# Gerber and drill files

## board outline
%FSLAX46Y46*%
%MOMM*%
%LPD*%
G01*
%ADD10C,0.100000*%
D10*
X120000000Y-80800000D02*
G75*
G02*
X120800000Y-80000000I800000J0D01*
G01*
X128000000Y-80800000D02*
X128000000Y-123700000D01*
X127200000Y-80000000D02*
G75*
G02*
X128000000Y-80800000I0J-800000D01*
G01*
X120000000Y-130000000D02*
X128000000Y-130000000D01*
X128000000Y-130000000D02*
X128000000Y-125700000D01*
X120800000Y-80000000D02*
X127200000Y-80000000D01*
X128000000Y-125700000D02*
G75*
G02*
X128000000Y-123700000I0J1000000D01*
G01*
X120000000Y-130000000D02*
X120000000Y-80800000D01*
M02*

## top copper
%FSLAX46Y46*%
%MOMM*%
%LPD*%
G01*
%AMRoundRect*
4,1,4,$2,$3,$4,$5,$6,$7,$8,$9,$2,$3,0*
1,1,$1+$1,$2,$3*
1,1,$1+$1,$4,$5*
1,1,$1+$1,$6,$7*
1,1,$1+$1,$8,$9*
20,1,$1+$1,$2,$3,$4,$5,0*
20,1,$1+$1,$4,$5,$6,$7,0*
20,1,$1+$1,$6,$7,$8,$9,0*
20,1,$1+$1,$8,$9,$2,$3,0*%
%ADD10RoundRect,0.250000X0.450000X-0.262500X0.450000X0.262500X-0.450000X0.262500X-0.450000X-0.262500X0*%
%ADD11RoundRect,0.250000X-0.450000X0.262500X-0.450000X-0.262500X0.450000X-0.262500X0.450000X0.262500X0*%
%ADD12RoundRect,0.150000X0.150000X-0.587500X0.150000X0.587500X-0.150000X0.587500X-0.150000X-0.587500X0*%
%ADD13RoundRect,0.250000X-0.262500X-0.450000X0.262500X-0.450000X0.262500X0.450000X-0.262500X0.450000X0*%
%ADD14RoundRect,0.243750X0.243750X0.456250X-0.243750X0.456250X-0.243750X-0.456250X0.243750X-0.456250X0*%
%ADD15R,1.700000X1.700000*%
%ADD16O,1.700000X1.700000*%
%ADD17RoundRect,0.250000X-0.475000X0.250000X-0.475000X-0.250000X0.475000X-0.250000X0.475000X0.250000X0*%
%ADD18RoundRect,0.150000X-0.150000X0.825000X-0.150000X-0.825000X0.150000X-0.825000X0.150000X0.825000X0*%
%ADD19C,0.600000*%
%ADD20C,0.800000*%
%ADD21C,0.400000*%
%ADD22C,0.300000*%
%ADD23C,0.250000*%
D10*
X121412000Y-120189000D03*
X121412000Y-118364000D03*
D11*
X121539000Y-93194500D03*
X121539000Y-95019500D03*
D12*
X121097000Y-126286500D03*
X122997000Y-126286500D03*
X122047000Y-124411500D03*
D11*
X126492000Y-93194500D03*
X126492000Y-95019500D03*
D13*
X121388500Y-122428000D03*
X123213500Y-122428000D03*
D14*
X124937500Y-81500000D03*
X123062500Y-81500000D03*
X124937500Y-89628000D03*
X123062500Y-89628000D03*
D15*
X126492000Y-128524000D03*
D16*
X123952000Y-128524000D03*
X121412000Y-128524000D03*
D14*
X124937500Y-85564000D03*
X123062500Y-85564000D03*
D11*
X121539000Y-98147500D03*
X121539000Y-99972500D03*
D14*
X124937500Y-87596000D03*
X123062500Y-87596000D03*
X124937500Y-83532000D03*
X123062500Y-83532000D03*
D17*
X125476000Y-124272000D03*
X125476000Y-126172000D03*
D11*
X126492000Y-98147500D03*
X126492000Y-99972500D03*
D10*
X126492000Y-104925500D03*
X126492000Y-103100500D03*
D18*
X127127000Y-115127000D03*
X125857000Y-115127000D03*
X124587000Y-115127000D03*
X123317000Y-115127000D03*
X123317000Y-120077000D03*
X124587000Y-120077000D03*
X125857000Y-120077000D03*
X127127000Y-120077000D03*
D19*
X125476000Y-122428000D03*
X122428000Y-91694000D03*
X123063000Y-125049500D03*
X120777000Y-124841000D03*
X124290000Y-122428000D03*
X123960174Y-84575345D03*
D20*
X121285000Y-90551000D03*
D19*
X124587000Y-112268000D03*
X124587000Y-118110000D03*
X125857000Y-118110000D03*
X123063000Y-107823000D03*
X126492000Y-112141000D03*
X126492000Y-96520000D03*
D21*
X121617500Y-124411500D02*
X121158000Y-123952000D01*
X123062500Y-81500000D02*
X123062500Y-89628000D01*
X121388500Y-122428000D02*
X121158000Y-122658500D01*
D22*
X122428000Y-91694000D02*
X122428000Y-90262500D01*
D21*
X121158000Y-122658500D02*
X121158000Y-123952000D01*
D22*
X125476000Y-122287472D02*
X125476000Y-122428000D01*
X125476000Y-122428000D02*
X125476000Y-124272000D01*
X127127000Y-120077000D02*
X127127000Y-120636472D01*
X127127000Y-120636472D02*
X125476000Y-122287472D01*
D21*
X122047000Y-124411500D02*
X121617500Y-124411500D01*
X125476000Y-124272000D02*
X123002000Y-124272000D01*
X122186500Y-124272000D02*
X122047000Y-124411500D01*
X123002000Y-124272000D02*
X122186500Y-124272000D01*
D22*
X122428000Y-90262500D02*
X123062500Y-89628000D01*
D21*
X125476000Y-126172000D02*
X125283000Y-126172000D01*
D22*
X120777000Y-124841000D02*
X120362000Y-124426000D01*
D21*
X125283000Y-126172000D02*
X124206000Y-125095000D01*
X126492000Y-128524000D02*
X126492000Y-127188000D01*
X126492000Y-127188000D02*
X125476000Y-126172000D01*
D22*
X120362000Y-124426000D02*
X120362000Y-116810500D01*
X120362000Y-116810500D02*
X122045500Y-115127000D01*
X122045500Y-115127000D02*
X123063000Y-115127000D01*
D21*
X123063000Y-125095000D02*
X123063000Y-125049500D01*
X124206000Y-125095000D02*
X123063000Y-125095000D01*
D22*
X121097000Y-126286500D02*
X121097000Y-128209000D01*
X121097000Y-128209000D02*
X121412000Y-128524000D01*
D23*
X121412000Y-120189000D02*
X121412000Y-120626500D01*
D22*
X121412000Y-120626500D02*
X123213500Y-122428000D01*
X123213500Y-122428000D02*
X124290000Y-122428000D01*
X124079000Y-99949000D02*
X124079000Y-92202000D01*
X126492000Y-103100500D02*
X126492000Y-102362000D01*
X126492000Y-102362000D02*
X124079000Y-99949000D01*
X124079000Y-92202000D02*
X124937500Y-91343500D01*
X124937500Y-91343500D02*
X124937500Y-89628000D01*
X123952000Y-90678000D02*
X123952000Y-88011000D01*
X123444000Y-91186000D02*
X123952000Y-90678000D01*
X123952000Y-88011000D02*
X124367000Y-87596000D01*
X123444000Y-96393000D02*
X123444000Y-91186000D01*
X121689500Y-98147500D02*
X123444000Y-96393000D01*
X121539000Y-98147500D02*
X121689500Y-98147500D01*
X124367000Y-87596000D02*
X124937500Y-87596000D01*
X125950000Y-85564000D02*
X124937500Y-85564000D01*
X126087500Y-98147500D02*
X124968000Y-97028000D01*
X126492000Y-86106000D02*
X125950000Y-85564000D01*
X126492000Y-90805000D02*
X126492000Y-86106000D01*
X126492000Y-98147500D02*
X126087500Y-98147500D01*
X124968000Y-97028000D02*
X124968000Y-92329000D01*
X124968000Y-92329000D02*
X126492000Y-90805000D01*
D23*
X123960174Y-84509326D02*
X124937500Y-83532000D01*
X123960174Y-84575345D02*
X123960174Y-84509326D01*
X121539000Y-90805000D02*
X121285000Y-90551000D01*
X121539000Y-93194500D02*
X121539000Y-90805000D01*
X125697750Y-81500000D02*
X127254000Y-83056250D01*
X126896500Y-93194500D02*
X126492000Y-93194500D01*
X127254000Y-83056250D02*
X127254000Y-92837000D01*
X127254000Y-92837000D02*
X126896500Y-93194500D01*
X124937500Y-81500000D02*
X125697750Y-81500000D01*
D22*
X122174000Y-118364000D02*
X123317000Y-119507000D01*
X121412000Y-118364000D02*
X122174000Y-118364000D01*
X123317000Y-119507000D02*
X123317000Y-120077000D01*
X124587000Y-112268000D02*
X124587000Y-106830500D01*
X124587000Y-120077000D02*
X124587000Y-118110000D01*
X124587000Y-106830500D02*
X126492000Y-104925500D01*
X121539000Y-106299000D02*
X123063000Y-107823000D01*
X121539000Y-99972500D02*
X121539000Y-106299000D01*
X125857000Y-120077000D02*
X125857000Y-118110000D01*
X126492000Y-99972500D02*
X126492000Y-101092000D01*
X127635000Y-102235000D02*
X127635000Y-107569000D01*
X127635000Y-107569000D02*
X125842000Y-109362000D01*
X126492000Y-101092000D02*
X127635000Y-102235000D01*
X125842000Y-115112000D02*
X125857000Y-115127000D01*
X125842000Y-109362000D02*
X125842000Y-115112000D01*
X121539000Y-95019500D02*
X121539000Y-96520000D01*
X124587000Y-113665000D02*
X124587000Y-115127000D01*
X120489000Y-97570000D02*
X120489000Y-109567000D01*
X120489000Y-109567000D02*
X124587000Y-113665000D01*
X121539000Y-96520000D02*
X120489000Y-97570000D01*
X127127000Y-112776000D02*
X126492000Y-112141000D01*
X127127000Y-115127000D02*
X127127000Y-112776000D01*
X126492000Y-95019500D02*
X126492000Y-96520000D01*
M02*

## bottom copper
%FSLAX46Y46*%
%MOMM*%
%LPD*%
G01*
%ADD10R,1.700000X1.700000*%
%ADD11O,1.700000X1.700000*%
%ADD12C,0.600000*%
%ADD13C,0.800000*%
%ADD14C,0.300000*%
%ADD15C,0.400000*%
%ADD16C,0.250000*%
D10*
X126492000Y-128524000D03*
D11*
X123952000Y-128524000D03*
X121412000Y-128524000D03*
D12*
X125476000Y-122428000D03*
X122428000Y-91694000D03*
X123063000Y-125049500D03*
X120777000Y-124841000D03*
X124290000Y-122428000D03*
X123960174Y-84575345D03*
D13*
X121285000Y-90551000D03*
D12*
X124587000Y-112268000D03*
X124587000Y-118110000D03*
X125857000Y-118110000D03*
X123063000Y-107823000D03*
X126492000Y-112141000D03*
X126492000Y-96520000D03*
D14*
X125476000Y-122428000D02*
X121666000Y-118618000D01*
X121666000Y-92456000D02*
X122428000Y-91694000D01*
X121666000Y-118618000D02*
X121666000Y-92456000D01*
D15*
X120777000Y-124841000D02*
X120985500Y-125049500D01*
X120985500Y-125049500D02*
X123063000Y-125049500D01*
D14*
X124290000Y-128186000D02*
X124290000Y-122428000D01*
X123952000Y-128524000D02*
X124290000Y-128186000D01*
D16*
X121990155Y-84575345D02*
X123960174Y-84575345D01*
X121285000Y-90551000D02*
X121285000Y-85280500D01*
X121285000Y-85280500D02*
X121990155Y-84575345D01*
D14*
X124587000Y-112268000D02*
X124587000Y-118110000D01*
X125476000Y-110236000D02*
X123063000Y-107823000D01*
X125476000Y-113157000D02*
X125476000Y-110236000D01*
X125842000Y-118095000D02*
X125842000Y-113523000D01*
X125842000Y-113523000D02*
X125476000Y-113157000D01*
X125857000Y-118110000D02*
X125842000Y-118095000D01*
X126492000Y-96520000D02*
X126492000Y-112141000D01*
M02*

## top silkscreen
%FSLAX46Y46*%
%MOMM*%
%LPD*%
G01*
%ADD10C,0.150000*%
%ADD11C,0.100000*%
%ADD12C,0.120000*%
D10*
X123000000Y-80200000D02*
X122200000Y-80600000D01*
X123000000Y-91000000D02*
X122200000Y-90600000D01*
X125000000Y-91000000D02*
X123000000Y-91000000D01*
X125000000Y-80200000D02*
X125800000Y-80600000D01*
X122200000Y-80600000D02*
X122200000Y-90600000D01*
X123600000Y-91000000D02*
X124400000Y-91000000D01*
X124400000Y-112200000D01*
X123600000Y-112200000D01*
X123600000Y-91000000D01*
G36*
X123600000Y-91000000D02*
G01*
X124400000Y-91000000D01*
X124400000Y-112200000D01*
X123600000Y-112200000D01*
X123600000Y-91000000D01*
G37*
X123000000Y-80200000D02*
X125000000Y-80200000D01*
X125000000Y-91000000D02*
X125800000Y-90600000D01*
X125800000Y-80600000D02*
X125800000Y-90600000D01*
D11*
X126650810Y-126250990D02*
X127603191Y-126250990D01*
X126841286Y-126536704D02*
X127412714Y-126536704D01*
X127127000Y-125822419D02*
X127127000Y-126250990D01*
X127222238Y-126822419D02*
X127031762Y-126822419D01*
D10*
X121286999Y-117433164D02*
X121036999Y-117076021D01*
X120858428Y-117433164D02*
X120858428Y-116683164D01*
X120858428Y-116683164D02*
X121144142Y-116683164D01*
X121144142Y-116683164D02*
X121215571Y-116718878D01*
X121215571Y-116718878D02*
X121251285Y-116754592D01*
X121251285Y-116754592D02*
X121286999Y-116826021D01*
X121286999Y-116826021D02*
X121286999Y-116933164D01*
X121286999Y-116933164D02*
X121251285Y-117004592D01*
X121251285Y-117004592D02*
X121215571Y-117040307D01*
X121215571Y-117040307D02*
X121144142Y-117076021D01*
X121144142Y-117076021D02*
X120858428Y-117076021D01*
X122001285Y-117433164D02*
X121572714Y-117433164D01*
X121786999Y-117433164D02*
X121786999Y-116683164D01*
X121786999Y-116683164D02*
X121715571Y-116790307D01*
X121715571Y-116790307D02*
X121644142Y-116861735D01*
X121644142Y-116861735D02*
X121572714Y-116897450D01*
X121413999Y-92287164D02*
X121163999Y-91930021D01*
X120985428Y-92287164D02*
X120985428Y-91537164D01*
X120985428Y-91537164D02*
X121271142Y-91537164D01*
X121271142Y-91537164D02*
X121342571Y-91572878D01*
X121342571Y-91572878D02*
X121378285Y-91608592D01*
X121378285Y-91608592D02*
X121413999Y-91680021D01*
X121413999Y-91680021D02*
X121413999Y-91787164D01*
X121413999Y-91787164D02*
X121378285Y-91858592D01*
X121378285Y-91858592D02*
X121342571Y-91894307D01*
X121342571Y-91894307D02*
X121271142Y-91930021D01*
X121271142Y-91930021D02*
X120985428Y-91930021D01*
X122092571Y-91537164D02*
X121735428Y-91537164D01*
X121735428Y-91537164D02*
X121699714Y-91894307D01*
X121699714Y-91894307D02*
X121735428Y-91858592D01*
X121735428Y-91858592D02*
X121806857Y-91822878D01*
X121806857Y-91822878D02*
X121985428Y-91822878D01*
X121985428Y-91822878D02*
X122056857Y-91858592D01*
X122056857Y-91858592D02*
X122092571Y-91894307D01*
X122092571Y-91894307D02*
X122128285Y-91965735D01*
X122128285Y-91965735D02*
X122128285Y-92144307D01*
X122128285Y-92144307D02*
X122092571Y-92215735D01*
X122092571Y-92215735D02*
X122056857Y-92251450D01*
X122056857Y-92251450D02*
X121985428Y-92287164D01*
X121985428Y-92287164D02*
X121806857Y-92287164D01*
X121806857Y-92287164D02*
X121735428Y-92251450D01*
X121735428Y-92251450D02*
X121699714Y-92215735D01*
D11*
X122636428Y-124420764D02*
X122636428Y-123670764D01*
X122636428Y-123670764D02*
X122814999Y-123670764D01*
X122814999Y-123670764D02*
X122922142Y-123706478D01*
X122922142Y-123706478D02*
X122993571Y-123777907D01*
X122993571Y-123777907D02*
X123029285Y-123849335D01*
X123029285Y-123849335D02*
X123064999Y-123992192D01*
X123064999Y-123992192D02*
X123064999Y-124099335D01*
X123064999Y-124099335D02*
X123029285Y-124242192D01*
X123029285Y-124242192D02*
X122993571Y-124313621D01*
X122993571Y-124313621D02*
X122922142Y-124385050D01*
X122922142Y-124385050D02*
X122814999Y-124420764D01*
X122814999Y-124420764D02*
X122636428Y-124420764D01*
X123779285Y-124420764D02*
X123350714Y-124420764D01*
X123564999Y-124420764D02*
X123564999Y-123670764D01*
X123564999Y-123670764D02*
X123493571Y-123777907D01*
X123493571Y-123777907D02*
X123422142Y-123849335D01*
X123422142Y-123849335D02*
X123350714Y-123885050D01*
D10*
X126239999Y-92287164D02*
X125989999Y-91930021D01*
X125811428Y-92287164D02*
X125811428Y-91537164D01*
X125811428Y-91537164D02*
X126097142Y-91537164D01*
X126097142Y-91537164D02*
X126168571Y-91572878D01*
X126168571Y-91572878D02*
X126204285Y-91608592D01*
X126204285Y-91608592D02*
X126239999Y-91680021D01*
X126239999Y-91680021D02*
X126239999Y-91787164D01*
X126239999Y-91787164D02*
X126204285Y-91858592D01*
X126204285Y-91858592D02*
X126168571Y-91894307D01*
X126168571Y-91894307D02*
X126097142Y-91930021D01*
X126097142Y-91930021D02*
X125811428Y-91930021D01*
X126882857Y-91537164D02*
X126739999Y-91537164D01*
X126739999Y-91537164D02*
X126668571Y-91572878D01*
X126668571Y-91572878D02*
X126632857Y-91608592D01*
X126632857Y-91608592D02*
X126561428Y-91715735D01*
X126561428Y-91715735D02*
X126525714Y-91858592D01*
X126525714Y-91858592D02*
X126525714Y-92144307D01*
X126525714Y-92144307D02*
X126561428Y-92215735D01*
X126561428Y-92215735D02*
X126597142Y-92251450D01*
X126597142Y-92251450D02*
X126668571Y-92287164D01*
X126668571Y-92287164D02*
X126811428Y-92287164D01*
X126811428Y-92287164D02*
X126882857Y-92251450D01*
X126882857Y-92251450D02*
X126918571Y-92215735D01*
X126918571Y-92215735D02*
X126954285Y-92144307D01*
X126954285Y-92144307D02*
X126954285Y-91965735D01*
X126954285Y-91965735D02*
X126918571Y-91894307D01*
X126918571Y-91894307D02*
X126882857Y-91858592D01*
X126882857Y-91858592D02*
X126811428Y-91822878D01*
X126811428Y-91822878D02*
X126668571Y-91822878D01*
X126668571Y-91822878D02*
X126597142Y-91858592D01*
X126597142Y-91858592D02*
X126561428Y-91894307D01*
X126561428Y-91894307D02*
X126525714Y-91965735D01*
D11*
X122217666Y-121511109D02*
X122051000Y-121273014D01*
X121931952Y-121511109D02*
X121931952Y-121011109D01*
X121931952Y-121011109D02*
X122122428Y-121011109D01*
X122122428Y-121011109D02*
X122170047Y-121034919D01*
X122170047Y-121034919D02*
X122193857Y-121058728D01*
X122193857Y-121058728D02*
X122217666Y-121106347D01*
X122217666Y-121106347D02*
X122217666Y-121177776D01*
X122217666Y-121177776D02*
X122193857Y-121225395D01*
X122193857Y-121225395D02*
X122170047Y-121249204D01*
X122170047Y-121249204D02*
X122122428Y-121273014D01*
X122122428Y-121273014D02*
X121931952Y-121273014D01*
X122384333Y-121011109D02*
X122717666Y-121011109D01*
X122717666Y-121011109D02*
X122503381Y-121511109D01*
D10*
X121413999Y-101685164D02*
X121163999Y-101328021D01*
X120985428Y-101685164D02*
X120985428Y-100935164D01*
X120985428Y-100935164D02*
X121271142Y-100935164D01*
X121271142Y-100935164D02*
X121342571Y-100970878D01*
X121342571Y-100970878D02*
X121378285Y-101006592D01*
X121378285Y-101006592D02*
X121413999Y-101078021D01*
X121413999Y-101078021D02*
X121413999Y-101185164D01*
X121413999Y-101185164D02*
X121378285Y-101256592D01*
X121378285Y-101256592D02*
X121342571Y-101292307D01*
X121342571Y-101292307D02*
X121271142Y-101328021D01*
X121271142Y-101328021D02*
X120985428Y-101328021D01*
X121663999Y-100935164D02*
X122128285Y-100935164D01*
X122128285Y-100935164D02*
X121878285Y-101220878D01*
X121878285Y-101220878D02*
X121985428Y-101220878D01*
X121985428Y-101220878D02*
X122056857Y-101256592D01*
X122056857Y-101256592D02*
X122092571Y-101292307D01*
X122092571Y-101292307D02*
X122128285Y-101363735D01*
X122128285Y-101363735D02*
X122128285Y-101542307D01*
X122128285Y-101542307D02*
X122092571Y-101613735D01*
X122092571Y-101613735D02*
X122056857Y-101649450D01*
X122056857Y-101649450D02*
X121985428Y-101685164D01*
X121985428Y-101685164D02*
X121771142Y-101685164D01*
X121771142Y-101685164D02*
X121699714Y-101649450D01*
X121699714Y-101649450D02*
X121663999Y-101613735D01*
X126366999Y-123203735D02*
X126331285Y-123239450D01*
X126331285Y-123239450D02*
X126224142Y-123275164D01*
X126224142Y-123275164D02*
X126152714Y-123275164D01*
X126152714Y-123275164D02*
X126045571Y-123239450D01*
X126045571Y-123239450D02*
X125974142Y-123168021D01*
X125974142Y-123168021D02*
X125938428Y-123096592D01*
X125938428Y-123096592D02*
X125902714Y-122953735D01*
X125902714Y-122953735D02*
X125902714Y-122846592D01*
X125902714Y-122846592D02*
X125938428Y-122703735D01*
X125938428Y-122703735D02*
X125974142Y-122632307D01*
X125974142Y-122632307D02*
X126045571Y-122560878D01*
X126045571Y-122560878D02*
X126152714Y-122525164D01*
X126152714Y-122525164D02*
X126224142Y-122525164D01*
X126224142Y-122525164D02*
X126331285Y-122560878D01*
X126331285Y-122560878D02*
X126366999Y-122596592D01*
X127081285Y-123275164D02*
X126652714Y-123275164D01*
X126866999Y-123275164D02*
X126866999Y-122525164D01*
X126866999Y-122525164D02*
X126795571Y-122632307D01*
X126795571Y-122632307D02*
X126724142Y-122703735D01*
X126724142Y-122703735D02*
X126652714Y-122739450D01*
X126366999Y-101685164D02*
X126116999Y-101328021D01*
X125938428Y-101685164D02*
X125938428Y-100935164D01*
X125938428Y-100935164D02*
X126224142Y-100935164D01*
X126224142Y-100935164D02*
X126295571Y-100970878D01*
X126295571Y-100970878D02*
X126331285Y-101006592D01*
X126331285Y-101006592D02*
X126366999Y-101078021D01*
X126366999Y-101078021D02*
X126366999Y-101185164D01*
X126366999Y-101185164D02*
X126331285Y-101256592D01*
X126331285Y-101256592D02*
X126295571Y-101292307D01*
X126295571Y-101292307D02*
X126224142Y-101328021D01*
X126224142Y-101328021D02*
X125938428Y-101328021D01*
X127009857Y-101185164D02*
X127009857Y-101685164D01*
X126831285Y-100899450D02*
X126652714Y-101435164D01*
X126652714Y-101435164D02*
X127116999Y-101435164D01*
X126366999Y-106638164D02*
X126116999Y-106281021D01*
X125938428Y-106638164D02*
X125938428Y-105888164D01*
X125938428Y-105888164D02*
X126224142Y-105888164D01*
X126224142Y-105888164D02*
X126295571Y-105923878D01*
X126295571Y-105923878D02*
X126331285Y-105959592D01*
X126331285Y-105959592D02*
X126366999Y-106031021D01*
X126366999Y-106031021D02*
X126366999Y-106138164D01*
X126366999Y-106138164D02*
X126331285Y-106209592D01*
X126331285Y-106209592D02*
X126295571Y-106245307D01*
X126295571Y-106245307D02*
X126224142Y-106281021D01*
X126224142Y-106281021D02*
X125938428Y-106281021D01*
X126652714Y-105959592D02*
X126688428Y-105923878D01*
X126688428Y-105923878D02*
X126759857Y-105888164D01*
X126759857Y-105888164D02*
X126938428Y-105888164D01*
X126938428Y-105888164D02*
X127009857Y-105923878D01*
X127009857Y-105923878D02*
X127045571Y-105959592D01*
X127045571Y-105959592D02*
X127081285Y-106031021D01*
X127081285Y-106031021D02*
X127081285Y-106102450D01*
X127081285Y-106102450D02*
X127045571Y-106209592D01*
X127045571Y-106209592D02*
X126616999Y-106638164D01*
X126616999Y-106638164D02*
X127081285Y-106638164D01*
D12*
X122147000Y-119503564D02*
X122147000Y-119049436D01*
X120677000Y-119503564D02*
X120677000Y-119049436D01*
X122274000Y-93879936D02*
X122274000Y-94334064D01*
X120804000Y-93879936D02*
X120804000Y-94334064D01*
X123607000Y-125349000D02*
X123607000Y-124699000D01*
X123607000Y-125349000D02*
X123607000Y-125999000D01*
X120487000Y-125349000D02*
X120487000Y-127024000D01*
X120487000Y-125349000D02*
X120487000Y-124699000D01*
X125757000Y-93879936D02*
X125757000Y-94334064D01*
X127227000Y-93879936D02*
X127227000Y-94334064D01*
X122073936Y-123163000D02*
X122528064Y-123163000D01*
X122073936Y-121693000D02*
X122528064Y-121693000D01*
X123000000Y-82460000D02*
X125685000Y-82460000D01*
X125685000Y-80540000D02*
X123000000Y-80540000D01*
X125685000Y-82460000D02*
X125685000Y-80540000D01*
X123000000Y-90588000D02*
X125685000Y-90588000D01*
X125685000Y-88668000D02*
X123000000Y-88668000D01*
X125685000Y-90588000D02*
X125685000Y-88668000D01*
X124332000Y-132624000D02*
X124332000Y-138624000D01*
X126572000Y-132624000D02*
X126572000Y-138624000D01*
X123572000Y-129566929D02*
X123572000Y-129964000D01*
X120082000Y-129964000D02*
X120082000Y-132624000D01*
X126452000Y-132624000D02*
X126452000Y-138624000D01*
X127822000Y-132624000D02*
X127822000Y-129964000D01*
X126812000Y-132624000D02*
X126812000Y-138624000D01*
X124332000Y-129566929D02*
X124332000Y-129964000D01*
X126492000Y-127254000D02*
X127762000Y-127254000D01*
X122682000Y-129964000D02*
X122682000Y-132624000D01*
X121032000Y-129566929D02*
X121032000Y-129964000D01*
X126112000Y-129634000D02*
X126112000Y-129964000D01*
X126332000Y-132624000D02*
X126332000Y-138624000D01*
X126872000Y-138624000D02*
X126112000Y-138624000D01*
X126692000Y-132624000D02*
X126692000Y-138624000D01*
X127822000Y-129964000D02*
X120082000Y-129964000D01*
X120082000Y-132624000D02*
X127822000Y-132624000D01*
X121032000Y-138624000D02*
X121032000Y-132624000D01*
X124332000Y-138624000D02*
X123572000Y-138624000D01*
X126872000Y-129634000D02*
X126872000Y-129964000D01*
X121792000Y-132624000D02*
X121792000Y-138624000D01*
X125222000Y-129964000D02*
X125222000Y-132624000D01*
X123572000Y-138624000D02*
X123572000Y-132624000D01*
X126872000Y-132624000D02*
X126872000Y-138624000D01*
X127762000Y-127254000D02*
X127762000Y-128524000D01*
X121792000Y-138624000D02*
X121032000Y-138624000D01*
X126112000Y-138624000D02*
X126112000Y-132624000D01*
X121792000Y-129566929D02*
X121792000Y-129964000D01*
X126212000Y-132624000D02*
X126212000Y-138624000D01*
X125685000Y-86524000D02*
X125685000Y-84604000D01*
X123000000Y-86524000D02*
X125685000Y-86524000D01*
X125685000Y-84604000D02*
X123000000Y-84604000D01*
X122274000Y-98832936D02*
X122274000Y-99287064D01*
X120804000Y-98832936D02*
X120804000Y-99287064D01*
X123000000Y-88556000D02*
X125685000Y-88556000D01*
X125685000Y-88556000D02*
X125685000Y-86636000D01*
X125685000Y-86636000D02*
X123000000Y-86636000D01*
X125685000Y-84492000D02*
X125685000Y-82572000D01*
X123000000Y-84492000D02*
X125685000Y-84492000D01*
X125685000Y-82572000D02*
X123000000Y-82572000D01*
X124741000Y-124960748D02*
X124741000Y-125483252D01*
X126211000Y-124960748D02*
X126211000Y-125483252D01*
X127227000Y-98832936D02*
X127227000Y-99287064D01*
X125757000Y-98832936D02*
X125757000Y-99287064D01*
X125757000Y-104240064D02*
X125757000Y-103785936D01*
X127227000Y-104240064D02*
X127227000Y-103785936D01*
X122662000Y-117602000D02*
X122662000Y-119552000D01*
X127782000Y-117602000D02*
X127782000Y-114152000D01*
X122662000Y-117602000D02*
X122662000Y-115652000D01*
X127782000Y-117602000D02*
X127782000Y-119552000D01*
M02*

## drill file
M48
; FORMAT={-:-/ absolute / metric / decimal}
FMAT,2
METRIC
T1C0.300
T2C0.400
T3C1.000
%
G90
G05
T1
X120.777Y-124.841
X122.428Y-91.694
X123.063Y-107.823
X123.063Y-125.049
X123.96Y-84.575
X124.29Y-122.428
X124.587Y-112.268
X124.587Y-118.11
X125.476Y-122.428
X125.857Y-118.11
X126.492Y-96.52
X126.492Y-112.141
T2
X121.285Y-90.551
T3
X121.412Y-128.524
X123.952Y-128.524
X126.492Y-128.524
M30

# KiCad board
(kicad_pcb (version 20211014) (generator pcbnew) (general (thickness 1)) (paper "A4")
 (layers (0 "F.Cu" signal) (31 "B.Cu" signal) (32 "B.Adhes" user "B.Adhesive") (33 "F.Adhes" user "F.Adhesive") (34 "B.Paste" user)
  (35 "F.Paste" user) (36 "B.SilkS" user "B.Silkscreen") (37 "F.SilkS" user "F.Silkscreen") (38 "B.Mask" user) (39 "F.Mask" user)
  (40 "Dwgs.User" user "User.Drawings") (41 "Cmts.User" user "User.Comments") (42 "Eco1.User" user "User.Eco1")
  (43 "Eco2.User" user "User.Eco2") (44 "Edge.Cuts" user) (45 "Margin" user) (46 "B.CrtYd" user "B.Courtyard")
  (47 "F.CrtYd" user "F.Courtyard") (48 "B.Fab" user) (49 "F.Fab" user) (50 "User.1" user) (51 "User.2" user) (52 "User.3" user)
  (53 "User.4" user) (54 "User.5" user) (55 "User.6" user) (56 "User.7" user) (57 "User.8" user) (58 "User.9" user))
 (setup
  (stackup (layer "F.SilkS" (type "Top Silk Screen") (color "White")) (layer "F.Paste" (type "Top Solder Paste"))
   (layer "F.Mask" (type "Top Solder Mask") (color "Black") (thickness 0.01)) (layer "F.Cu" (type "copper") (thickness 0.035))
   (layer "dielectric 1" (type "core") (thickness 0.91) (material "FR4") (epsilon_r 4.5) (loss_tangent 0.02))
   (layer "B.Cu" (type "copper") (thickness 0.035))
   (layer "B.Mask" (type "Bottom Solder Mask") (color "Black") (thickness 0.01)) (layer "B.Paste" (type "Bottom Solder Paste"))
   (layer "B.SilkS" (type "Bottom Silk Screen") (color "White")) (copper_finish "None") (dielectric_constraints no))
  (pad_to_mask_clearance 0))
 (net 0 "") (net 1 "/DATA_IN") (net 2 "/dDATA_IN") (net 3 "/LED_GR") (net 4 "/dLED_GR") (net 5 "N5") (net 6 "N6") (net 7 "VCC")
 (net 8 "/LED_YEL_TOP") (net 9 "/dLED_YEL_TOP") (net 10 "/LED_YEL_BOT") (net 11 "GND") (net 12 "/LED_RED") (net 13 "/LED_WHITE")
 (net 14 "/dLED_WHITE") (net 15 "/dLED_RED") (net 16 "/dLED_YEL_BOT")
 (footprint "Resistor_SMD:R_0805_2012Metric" (layer "F.Cu") (at 121.412 119.2765 90)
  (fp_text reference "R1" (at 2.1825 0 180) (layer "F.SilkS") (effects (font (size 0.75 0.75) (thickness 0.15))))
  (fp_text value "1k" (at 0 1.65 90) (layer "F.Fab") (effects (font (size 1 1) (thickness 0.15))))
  (fp_line (start -0.227064 0.735) (end 0.227064 0.735) (layer "F.SilkS") (width 0.12))
  (fp_line (start -0.227064 -0.735) (end 0.227064 -0.735) (layer "F.SilkS") (width 0.12))
  (pad "1" smd roundrect (at -0.9125 0 90) (size 1.025 1.4) (layers "F.Cu" "F.Paste" "F.Mask") (roundrect_rratio 0.243902)
   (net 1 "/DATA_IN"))
  (pad "2" smd roundrect (at 0.9125 0 90) (size 1.025 1.4) (layers "F.Cu" "F.Paste" "F.Mask") (roundrect_rratio 0.243902)
   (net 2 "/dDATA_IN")))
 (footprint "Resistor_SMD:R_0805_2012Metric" (layer "F.Cu") (at 121.539 94.107 -90)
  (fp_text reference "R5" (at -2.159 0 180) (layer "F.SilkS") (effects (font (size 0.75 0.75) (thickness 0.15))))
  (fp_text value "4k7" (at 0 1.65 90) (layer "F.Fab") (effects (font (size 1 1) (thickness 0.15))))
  (fp_line (start -0.227064 -0.735) (end 0.227064 -0.735) (layer "F.SilkS") (width 0.12))
  (fp_line (start -0.227064 0.735) (end 0.227064 0.735) (layer "F.SilkS") (width 0.12))
  (pad "1" smd roundrect (at -0.9125 0 270) (size 1.025 1.4) (layers "F.Cu" "F.Paste" "F.Mask") (roundrect_rratio 0.243902)
   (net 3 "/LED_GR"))
  (pad "2" smd roundrect (at 0.9125 0 270) (size 1.025 1.4) (layers "F.Cu" "F.Paste" "F.Mask") (roundrect_rratio 0.243902)
   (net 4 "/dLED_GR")))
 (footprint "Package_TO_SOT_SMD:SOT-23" (layer "F.Cu") (at 122.047 125.349 90)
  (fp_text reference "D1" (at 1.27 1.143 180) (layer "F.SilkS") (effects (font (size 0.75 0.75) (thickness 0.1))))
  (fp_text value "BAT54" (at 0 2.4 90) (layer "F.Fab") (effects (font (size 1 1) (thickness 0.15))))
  (fp_line (start 0 1.56) (end 0.65 1.56) (layer "F.SilkS") (width 0.12))
  (fp_line (start 0 1.56) (end -0.65 1.56) (layer "F.SilkS") (width 0.12))
  (fp_line (start 0 -1.56) (end -1.675 -1.56) (layer "F.SilkS") (width 0.12))
  (fp_line (start 0 -1.56) (end 0.65 -1.56) (layer "F.SilkS") (width 0.12))
  (pad "1" smd roundrect (at -0.9375 -0.95 90) (size 1.475 0.6) (layers "F.Cu" "F.Paste" "F.Mask") (roundrect_rratio 0.25) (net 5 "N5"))
  (pad "2" smd roundrect (at -0.9375 0.95 90) (size 1.475 0.6) (layers "F.Cu" "F.Paste" "F.Mask") (roundrect_rratio 0.25) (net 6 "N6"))
  (pad "3" smd roundrect (at 0.9375 0 90) (size 1.475 0.6) (layers "F.Cu" "F.Paste" "F.Mask") (roundrect_rratio 0.25) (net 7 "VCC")))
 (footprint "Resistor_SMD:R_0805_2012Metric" (layer "F.Cu") (at 126.492 94.107 -90)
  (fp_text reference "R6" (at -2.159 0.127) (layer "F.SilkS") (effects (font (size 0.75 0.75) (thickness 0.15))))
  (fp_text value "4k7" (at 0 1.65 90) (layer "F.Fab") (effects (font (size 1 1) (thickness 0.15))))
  (fp_line (start -0.227064 0.735) (end 0.227064 0.735) (layer "F.SilkS") (width 0.12))
  (fp_line (start -0.227064 -0.735) (end 0.227064 -0.735) (layer "F.SilkS") (width 0.12))
  (pad "1" smd roundrect (at -0.9125 0 270) (size 1.025 1.4) (layers "F.Cu" "F.Paste" "F.Mask") (roundrect_rratio 0.243902)
   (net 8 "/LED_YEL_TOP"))
  (pad "2" smd roundrect (at 0.9125 0 270) (size 1.025 1.4) (layers "F.Cu" "F.Paste" "F.Mask") (roundrect_rratio 0.243902)
   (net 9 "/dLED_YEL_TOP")))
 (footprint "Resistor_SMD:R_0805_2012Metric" (layer "F.Cu") (at 122.301 122.428)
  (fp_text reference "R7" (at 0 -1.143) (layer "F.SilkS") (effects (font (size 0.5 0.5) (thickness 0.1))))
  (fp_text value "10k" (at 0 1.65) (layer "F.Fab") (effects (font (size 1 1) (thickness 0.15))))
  (fp_line (start -0.227064 0.735) (end 0.227064 0.735) (layer "F.SilkS") (width 0.12))
  (fp_line (start -0.227064 -0.735) (end 0.227064 -0.735) (layer "F.SilkS") (width 0.12))
  (pad "1" smd roundrect (at -0.9125 0) (size 1.025 1.4) (layers "F.Cu" "F.Paste" "F.Mask") (roundrect_rratio 0.243902) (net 7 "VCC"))
  (pad "2" smd roundrect (at 0.9125 0) (size 1.025 1.4) (layers "F.Cu" "F.Paste" "F.Mask") (roundrect_rratio 0.243902) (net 1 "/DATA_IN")))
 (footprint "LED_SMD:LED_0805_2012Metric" (layer "F.Cu") (at 124 81.5 180)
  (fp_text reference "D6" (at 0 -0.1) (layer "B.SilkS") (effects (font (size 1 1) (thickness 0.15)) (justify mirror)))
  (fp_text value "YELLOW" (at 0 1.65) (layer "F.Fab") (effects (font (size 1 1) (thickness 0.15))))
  (fp_line (start 1 -0.96) (end -1.685 -0.96) (layer "F.SilkS") (width 0.12))
  (fp_line (start -1.685 0.96) (end 1 0.96) (layer "F.SilkS") (width 0.12))
  (fp_line (start -1.685 -0.96) (end -1.685 0.96) (layer "F.SilkS") (width 0.12))
  (pad "1" smd roundrect (at -0.9375 0 180) (size 0.975 1.4) (layers "F.Cu" "F.Paste" "F.Mask") (roundrect_rratio 0.25)
   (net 8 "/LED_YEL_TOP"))
  (pad "2" smd roundrect (at 0.9375 0 180) (size 0.975 1.4) (layers "F.Cu" "F.Paste" "F.Mask") (roundrect_rratio 0.25) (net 7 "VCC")))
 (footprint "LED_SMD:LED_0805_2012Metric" (layer "F.Cu") (at 124 89.628 180)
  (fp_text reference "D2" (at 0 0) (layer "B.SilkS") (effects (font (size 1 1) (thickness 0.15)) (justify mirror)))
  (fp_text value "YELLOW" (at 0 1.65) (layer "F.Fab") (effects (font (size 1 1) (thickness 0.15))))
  (fp_line (start 1 -0.96) (end -1.685 -0.96) (layer "F.SilkS") (width 0.12))
  (fp_line (start -1.685 0.96) (end 1 0.96) (layer "F.SilkS") (width 0.12))
  (fp_line (start -1.685 -0.96) (end -1.685 0.96) (layer "F.SilkS") (width 0.12))
  (pad "1" smd roundrect (at -0.9375 0 180) (size 0.975 1.4) (layers "F.Cu" "F.Paste" "F.Mask") (roundrect_rratio 0.25)
   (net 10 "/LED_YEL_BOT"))
  (pad "2" smd roundrect (at 0.9375 0 180) (size 0.975 1.4) (layers "F.Cu" "F.Paste" "F.Mask") (roundrect_rratio 0.25) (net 7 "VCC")))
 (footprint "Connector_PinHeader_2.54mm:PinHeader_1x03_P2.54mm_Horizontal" (layer "F.Cu") (at 126.492 128.524 -90)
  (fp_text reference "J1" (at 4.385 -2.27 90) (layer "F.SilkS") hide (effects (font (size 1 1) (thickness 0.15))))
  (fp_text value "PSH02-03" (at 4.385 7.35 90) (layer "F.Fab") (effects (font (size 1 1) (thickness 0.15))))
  (fp_line (start 4.1 2.16) (end 10.1 2.16) (layer "F.SilkS") (width 0.12))
  (fp_line (start 4.1 -0.08) (end 10.1 -0.08) (layer "F.SilkS") (width 0.12))
  (fp_line (start 1.042929 2.92) (end 1.44 2.92) (layer "F.SilkS") (width 0.12))
  (fp_line (start 1.44 6.41) (end 4.1 6.41) (layer "F.SilkS") (width 0.12))
  (fp_line (start 4.1 0.04) (end 10.1 0.04) (layer "F.SilkS") (width 0.12))
  (fp_line (start 4.1 -1.33) (end 1.44 -1.33) (layer "F.SilkS") (width 0.12))
  (fp_line (start 4.1 -0.32) (end 10.1 -0.32) (layer "F.SilkS") (width 0.12))
  (fp_line (start 1.042929 2.16) (end 1.44 2.16) (layer "F.SilkS") (width 0.12))
  (fp_line (start -1.27 0) (end -1.27 -1.27) (layer "F.SilkS") (width 0.12))
  (fp_line (start 1.44 3.81) (end 4.1 3.81) (layer "F.SilkS") (width 0.12))
  (fp_line (start 1.042929 5.46) (end 1.44 5.46) (layer "F.SilkS") (width 0.12))
  (fp_line (start 1.11 0.38) (end 1.44 0.38) (layer "F.SilkS") (width 0.12))
  (fp_line (start 4.1 0.16) (end 10.1 0.16) (layer "F.SilkS") (width 0.12))
  (fp_line (start 10.1 -0.38) (end 10.1 0.38) (layer "F.SilkS") (width 0.12))
  (fp_line (start 4.1 -0.2) (end 10.1 -0.2) (layer "F.SilkS") (width 0.12))
  (fp_line (start 1.44 -1.33) (end 1.44 6.41) (layer "F.SilkS") (width 0.12))
  (fp_line (start 4.1 6.41) (end 4.1 -1.33) (layer "F.SilkS") (width 0.12))
  (fp_line (start 10.1 5.46) (end 4.1 5.46) (layer "F.SilkS") (width 0.12))
  (fp_line (start 10.1 2.16) (end 10.1 2.92) (layer "F.SilkS") (width 0.12))
  (fp_line (start 1.11 -0.38) (end 1.44 -0.38) (layer "F.SilkS") (width 0.12))
  (fp_line (start 4.1 4.7) (end 10.1 4.7) (layer "F.SilkS") (width 0.12))
  (fp_line (start 1.44 1.27) (end 4.1 1.27) (layer "F.SilkS") (width 0.12))
  (fp_line (start 10.1 2.92) (end 4.1 2.92) (layer "F.SilkS") (width 0.12))
  (fp_line (start 4.1 -0.38) (end 10.1 -0.38) (layer "F.SilkS") (width 0.12))
  (fp_line (start -1.27 -1.27) (end 0 -1.27) (layer "F.SilkS") (width 0.12))
  (fp_line (start 10.1 4.7) (end 10.1 5.46) (layer "F.SilkS") (width 0.12))
  (fp_line (start 10.1 0.38) (end 4.1 0.38) (layer "F.SilkS") (width 0.12))
  (fp_line (start 1.042929 4.7) (end 1.44 4.7) (layer "F.SilkS") (width 0.12))
  (fp_line (start 4.1 0.28) (end 10.1 0.28) (layer "F.SilkS") (width 0.12))
  (pad "1" thru_hole rect (at 0 0 270) (size 1.7 1.7) (drill 1) (layers *.Cu *.Mask) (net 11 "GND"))
  (pad "2" thru_hole oval (at 0 2.54 270) (size 1.7 1.7) (drill 1) (layers *.Cu *.Mask) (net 1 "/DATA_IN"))
  (pad "3" thru_hole oval (at 0 5.08 270) (size 1.7 1.7) (drill 1) (layers *.Cu *.Mask) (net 5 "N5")))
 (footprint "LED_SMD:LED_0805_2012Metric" (layer "F.Cu") (at 124 85.564 180)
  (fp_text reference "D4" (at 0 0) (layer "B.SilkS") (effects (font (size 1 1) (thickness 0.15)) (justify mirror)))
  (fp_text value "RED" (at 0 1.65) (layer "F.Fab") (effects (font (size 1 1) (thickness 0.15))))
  (fp_line (start -1.685 -0.96) (end -1.685 0.96) (layer "F.SilkS") (width 0.12))
  (fp_line (start 1 -0.96) (end -1.685 -0.96) (layer "F.SilkS") (width 0.12))
  (fp_line (start -1.685 0.96) (end 1 0.96) (layer "F.SilkS") (width 0.12))
  (pad "1" smd roundrect (at -0.9375 0 180) (size 0.975 1.4) (layers "F.Cu" "F.Paste" "F.Mask") (roundrect_rratio 0.25) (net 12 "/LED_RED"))
  (pad "2" smd roundrect (at 0.9375 0 180) (size 0.975 1.4) (layers "F.Cu" "F.Paste" "F.Mask") (roundrect_rratio 0.25) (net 7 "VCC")))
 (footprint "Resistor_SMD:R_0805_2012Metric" (layer "F.Cu") (at 121.539 99.06 -90)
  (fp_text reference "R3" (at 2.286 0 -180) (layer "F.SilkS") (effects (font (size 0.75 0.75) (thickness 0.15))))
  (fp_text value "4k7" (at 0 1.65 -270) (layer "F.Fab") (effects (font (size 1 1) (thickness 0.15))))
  (fp_line (start -0.227064 -0.735) (end 0.227064 -0.735) (layer "F.SilkS") (width 0.12))
  (fp_line (start -0.227064 0.735) (end 0.227064 0.735) (layer "F.SilkS") (width 0.12))
  (pad "1" smd roundrect (at -0.9125 0 270) (size 1.025 1.4) (layers "F.Cu" "F.Paste" "F.Mask") (roundrect_rratio 0.243902)
   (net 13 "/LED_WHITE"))
  (pad "2" smd roundrect (at 0.9125 0 270) (size 1.025 1.4) (layers "F.Cu" "F.Paste" "F.Mask") (roundrect_rratio 0.243902)
   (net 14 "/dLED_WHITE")))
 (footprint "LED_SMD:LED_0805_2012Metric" (layer "F.Cu") (at 124 87.596 180)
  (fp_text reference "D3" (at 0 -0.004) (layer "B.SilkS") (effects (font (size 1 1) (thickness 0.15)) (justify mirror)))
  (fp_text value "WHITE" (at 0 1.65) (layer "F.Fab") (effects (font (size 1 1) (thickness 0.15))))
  (fp_line (start 1 -0.96) (end -1.685 -0.96) (layer "F.SilkS") (width 0.12))
  (fp_line (start -1.685 -0.96) (end -1.685 0.96) (layer "F.SilkS") (width 0.12))
  (fp_line (start -1.685 0.96) (end 1 0.96) (layer "F.SilkS") (width 0.12))
  (pad "1" smd roundrect (at -0.9375 0 180) (size 0.975 1.4) (layers "F.Cu" "F.Paste" "F.Mask") (roundrect_rratio 0.25)
   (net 13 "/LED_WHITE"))
  (pad "2" smd roundrect (at 0.9375 0 180) (size 0.975 1.4) (layers "F.Cu" "F.Paste" "F.Mask") (roundrect_rratio 0.25) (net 7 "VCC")))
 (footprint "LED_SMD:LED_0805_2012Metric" (layer "F.Cu") (at 124 83.532 180)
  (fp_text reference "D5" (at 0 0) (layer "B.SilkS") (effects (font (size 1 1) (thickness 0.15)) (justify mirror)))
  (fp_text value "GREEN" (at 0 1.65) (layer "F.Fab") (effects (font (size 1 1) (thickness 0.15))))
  (fp_line (start -1.685 -0.96) (end -1.685 0.96) (layer "F.SilkS") (width 0.12))
  (fp_line (start 1 -0.96) (end -1.685 -0.96) (layer "F.SilkS") (width 0.12))
  (fp_line (start -1.685 0.96) (end 1 0.96) (layer "F.SilkS") (width 0.12))
  (pad "1" smd roundrect (at -0.9375 0 180) (size 0.975 1.4) (layers "F.Cu" "F.Paste" "F.Mask") (roundrect_rratio 0.25) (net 3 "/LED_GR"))
  (pad "2" smd roundrect (at 0.9375 0 180) (size 0.975 1.4) (layers "F.Cu" "F.Paste" "F.Mask") (roundrect_rratio 0.25) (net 7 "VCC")))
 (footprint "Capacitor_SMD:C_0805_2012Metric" (layer "F.Cu") (at 125.476 125.222 -90)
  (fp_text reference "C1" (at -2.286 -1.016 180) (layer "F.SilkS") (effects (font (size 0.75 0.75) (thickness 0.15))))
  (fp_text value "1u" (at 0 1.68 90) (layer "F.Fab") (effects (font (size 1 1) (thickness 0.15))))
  (fp_line (start -0.261252 0.735) (end 0.261252 0.735) (layer "F.SilkS") (width 0.12))
  (fp_line (start -0.261252 -0.735) (end 0.261252 -0.735) (layer "F.SilkS") (width 0.12))
  (pad "1" smd roundrect (at -0.95 0 270) (size 1 1.45) (layers "F.Cu" "F.Paste" "F.Mask") (roundrect_rratio 0.25) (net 7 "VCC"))
  (pad "2" smd roundrect (at 0.95 0 270) (size 1 1.45) (layers "F.Cu" "F.Paste" "F.Mask") (roundrect_rratio 0.25) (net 11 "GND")))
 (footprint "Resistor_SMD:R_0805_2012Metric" (layer "F.Cu") (at 126.492 99.06 -90)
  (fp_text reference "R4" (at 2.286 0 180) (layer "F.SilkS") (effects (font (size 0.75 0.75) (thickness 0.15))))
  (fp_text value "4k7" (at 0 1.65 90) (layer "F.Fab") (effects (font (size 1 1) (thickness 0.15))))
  (fp_line (start -0.227064 -0.735) (end 0.227064 -0.735) (layer "F.SilkS") (width 0.12))
  (fp_line (start -0.227064 0.735) (end 0.227064 0.735) (layer "F.SilkS") (width 0.12))
  (pad "1" smd roundrect (at -0.9125 0 270) (size 1.025 1.4) (layers "F.Cu" "F.Paste" "F.Mask") (roundrect_rratio 0.243902)
   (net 12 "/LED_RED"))
  (pad "2" smd roundrect (at 0.9125 0 270) (size 1.025 1.4) (layers "F.Cu" "F.Paste" "F.Mask") (roundrect_rratio 0.243902)
   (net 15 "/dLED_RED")))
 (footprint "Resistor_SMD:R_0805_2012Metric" (layer "F.Cu") (at 126.492 104.013 90)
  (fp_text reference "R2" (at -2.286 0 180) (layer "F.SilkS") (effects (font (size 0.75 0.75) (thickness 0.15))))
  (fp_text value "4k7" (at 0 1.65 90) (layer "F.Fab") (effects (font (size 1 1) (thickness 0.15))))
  (fp_line (start -0.227064 -0.735) (end 0.227064 -0.735) (layer "F.SilkS") (width 0.12))
  (fp_line (start -0.227064 0.735) (end 0.227064 0.735) (layer "F.SilkS") (width 0.12))
  (pad "1" smd roundrect (at -0.9125 0 90) (size 1.025 1.4) (layers "F.Cu" "F.Paste" "F.Mask") (roundrect_rratio 0.243902)
   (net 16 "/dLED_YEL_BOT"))
  (pad "2" smd roundrect (at 0.9125 0 90) (size 1.025 1.4) (layers "F.Cu" "F.Paste" "F.Mask") (roundrect_rratio 0.243902)
   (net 10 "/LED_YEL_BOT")))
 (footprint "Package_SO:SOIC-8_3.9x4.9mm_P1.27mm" (layer "F.Cu") (at 125.222 117.602 -90)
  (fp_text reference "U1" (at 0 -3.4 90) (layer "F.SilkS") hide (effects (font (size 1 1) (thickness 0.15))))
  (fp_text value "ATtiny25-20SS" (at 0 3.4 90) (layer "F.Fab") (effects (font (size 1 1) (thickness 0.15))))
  (fp_line (start 0 2.56) (end 1.95 2.56) (layer "F.SilkS") (width 0.12))
  (fp_line (start 0 -2.56) (end -3.45 -2.56) (layer "F.SilkS") (width 0.12))
  (fp_line (start 0 2.56) (end -1.95 2.56) (layer "F.SilkS") (width 0.12))
  (fp_line (start 0 -2.56) (end 1.95 -2.56) (layer "F.SilkS") (width 0.12))
  (pad "1" smd roundrect (at -2.475 -1.905 270) (size 1.95 0.6) (layers "F.Cu" "F.Paste" "F.Mask") (roundrect_rratio 0.25)
   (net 9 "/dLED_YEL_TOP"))
  (pad "2" smd roundrect (at -2.475 -0.635 270) (size 1.95 0.6) (layers "F.Cu" "F.Paste" "F.Mask") (roundrect_rratio 0.25)
   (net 15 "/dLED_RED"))
  (pad "3" smd roundrect (at -2.475 0.635 270) (size 1.95 0.6) (layers "F.Cu" "F.Paste" "F.Mask") (roundrect_rratio 0.25) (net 4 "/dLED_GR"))
  (pad "4" smd roundrect (at -2.475 1.905 270) (size 1.95 0.6) (layers "F.Cu" "F.Paste" "F.Mask") (roundrect_rratio 0.25) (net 11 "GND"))
  (pad "5" smd roundrect (at 2.475 1.905 270) (size 1.95 0.6) (layers "F.Cu" "F.Paste" "F.Mask") (roundrect_rratio 0.25) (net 2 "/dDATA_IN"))
  (pad "6" smd roundrect (at 2.475 0.635 270) (size 1.95 0.6) (layers "F.Cu" "F.Paste" "F.Mask") (roundrect_rratio 0.25)
   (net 16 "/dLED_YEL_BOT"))
  (pad "7" smd roundrect (at 2.475 -0.635 270) (size 1.95 0.6) (layers "F.Cu" "F.Paste" "F.Mask") (roundrect_rratio 0.25)
   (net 14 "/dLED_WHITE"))
  (pad "8" smd roundrect (at 2.475 -1.905 270) (size 1.95 0.6) (layers "F.Cu" "F.Paste" "F.Mask") (roundrect_rratio 0.25) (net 7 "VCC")))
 (gr_line (start 123 80.2) (end 122.2 80.6) (layer "F.SilkS") (width 0.15))
 (gr_line (start 123 91) (end 122.2 90.6) (layer "F.SilkS") (width 0.15))
 (gr_line (start 125 91) (end 123 91) (layer "F.SilkS") (width 0.15))
 (gr_line (start 125 80.2) (end 125.8 80.6) (layer "F.SilkS") (width 0.15))
 (gr_line (start 122.2 80.6) (end 122.2 90.6) (layer "F.SilkS") (width 0.15))
 (gr_rect (start 123.6 91) (end 124.4 112.2) (layer "F.SilkS") (width 0.15) (fill solid))
 (gr_line (start 123 80.2) (end 125 80.2) (layer "F.SilkS") (width 0.15))
 (gr_line (start 125 91) (end 125.8 90.6) (layer "F.SilkS") (width 0.15))
 (gr_line (start 125.8 80.6) (end 125.8 90.6) (layer "F.SilkS") (width 0.15))
 (gr_arc (start 120 80.8) (mid 120.234315 80.234315) (end 120.8 80) (layer "Edge.Cuts") (width 0.1))
 (gr_line (start 128 80.8) (end 128 123.7) (layer "Edge.Cuts") (width 0.1))
 (gr_arc (start 127.2 80) (mid 127.765685 80.234315) (end 128 80.8) (layer "Edge.Cuts") (width 0.1))
 (gr_line (start 120 130) (end 128 130) (layer "Edge.Cuts") (width 0.1))
 (gr_line (start 128 130) (end 128 125.7) (layer "Edge.Cuts") (width 0.1))
 (gr_line (start 120.8 80) (end 127.2 80) (layer "Edge.Cuts") (width 0.1))
 (gr_arc (start 128 125.7) (mid 127 124.7) (end 128 123.7) (layer "Edge.Cuts") (width 0.1))
 (gr_line (start 120 130) (end 120 80.8) (layer "Edge.Cuts") (width 0.1))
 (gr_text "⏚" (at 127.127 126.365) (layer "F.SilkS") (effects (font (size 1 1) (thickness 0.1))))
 (segment (start 121.6175 124.4115) (end 121.158 123.952) (width 0.4) (layer "F.Cu") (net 7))
 (segment (start 123.0625 81.5) (end 123.0625 89.628) (width 0.4) (layer "F.Cu") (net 7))
 (segment (start 121.3885 122.428) (end 121.158 122.6585) (width 0.4) (layer "F.Cu") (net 7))
 (segment (start 122.428 91.694) (end 122.428 90.2625) (width 0.3) (layer "F.Cu") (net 7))
 (segment (start 121.158 122.6585) (end 121.158 123.952) (width 0.4) (layer "F.Cu") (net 7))
 (segment (start 125.476 122.287472) (end 125.476 122.428) (width 0.3) (layer "F.Cu") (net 7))
 (segment (start 125.476 122.428) (end 125.476 124.272) (width 0.3) (layer "F.Cu") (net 7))
 (segment (start 127.127 120.077) (end 127.127 120.636472) (width 0.3) (layer "F.Cu") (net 7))
 (segment (start 127.127 120.636472) (end 125.476 122.287472) (width 0.3) (layer "F.Cu") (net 7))
 (segment (start 122.047 124.4115) (end 121.6175 124.4115) (width 0.4) (layer "F.Cu") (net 7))
 (segment (start 125.476 124.272) (end 123.002 124.272) (width 0.4) (layer "F.Cu") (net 7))
 (segment (start 122.1865 124.272) (end 122.047 124.4115) (width 0.4) (layer "F.Cu") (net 7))
 (segment (start 123.002 124.272) (end 122.1865 124.272) (width 0.4) (layer "F.Cu") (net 7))
 (segment (start 122.428 90.2625) (end 123.0625 89.628) (width 0.3) (layer "F.Cu") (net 7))
 (via (at 125.476 122.428) (size 0.6) (drill 0.3) (layers "F.Cu" "B.Cu") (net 7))
 (via (at 122.428 91.694) (size 0.6) (drill 0.3) (layers "F.Cu" "B.Cu") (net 7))
 (segment (start 125.476 122.428) (end 121.666 118.618) (width 0.3) (layer "B.Cu") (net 7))
 (segment (start 121.666 92.456) (end 122.428 91.694) (width 0.3) (layer "B.Cu") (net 7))
 (segment (start 121.666 118.618) (end 121.666 92.456) (width 0.3) (layer "B.Cu") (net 7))
 (segment (start 125.476 126.172) (end 125.283 126.172) (width 0.4) (layer "F.Cu") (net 11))
 (segment (start 120.777 124.841) (end 120.362 124.426) (width 0.3) (layer "F.Cu") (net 11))
 (segment (start 125.283 126.172) (end 124.206 125.095) (width 0.4) (layer "F.Cu") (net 11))
 (segment (start 126.492 128.524) (end 126.492 127.188) (width 0.4) (layer "F.Cu") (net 11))
 (segment (start 126.492 127.188) (end 125.476 126.172) (width 0.4) (layer "F.Cu") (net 11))
 (segment (start 120.362 124.426) (end 120.362 116.8105) (width 0.3) (layer "F.Cu") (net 11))
 (segment (start 120.362 116.8105) (end 122.0455 115.127) (width 0.3) (layer "F.Cu") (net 11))
 (segment (start 122.0455 115.127) (end 123.063 115.127) (width 0.3) (layer "F.Cu") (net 11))
 (segment (start 123.063 125.095) (end 123.063 125.0495) (width 0.4) (layer "F.Cu") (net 11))
 (segment (start 124.206 125.095) (end 123.063 125.095) (width 0.4) (layer "F.Cu") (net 11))
 (via (at 123.063 125.0495) (size 0.6) (drill 0.3) (layers "F.Cu" "B.Cu") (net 11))
 (via (at 120.777 124.841) (size 0.6) (drill 0.3) (layers "F.Cu" "B.Cu") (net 11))
 (segment (start 120.777 124.841) (end 120.9855 125.0495) (width 0.4) (layer "B.Cu") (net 11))
 (segment (start 120.9855 125.0495) (end 123.063 125.0495) (width 0.4) (layer "B.Cu") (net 11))
 (segment (start 121.097 126.2865) (end 121.097 128.209) (width 0.3) (layer "F.Cu") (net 5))
 (segment (start 121.097 128.209) (end 121.412 128.524) (width 0.3) (layer "F.Cu") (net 5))
 (segment (start 121.412 120.189) (end 121.412 120.6265) (width 0.25) (layer "F.Cu") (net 1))
 (segment (start 121.412 120.6265) (end 123.2135 122.428) (width 0.3) (layer "F.Cu") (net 1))
 (segment (start 123.2135 122.428) (end 124.29 122.428) (width 0.3) (layer "F.Cu") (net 1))
 (via (at 124.29 122.428) (size 0.6) (drill 0.3) (layers "F.Cu" "B.Cu") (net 1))
 (segment (start 124.29 128.186) (end 124.29 122.428) (width 0.3) (layer "B.Cu") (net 1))
 (segment (start 123.952 128.524) (end 124.29 128.186) (width 0.3) (layer "B.Cu") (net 1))
 (segment (start 124.079 99.949) (end 124.079 92.202) (width 0.3) (layer "F.Cu") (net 10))
 (segment (start 126.492 103.1005) (end 126.492 102.362) (width 0.3) (layer "F.Cu") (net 10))
 (segment (start 126.492 102.362) (end 124.079 99.949) (width 0.3) (layer "F.Cu") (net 10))
 (segment (start 124.079 92.202) (end 124.9375 91.3435) (width 0.3) (layer "F.Cu") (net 10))
 (segment (start 124.9375 91.3435) (end 124.9375 89.628) (width 0.3) (layer "F.Cu") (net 10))
 (segment (start 123.952 90.678) (end 123.952 88.011) (width 0.3) (layer "F.Cu") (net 13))
 (segment (start 123.444 91.186) (end 123.952 90.678) (width 0.3) (layer "F.Cu") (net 13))
 (segment (start 123.952 88.011) (end 124.367 87.596) (width 0.3) (layer "F.Cu") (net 13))
 (segment (start 123.444 96.393) (end 123.444 91.186) (width 0.3) (layer "F.Cu") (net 13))
 (segment (start 121.6895 98.1475) (end 123.444 96.393) (width 0.3) (layer "F.Cu") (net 13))
 (segment (start 121.539 98.1475) (end 121.6895 98.1475) (width 0.3) (layer "F.Cu") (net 13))
 (segment (start 124.367 87.596) (end 124.9375 87.596) (width 0.3) (layer "F.Cu") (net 13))
 (segment (start 125.95 85.564) (end 124.9375 85.564) (width 0.3) (layer "F.Cu") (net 12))
 (segment (start 126.0875 98.1475) (end 124.968 97.028) (width 0.3) (layer "F.Cu") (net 12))
 (segment (start 126.492 86.106) (end 125.95 85.564) (width 0.3) (layer "F.Cu") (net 12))
 (segment (start 126.492 90.805) (end 126.492 86.106) (width 0.3) (layer "F.Cu") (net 12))
 (segment (start 126.492 98.1475) (end 126.0875 98.1475) (width 0.3) (layer "F.Cu") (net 12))
 (segment (start 124.968 97.028) (end 124.968 92.329) (width 0.3) (layer "F.Cu") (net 12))
 (segment (start 124.968 92.329) (end 126.492 90.805) (width 0.3) (layer "F.Cu") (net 12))
 (segment (start 123.960174 84.509326) (end 124.9375 83.532) (width 0.25) (layer "F.Cu") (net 3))
 (segment (start 123.960174 84.575345) (end 123.960174 84.509326) (width 0.25) (layer "F.Cu") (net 3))
 (segment (start 121.539 90.805) (end 121.285 90.551) (width 0.25) (layer "F.Cu") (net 3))
 (segment (start 121.539 93.1945) (end 121.539 90.805) (width 0.25) (layer "F.Cu") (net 3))
 (via (at 123.960174 84.575345) (size 0.6) (drill 0.3) (layers "F.Cu" "B.Cu") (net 3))
 (via (at 121.285 90.551) (size 0.8) (drill 0.4) (layers "F.Cu" "B.Cu") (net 3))
 (segment (start 121.990155 84.575345) (end 123.960174 84.575345) (width 0.25) (layer "B.Cu") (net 3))
 (segment (start 121.285 90.551) (end 121.285 85.2805) (width 0.25) (layer "B.Cu") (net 3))
 (segment (start 121.285 85.2805) (end 121.990155 84.575345) (width 0.25) (layer "B.Cu") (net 3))
 (segment (start 125.69775 81.5) (end 127.254 83.05625) (width 0.25) (layer "F.Cu") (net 8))
 (segment (start 126.8965 93.1945) (end 126.492 93.1945) (width 0.25) (layer "F.Cu") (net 8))
 (segment (start 127.254 83.05625) (end 127.254 92.837) (width 0.25) (layer "F.Cu") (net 8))
 (segment (start 127.254 92.837) (end 126.8965 93.1945) (width 0.25) (layer "F.Cu") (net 8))
 (segment (start 124.9375 81.5) (end 125.69775 81.5) (width 0.25) (layer "F.Cu") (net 8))
 (segment (start 122.174 118.364) (end 123.317 119.507) (width 0.3) (layer "F.Cu") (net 2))
 (segment (start 121.412 118.364) (end 122.174 118.364) (width 0.3) (layer "F.Cu") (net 2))
 (segment (start 123.317 119.507) (end 123.317 120.077) (width 0.3) (layer "F.Cu") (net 2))
 (segment (start 124.587 112.268) (end 124.587 106.8305) (width 0.3) (layer "F.Cu") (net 16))
 (segment (start 124.587 120.077) (end 124.587 118.11) (width 0.3) (layer "F.Cu") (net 16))
 (segment (start 124.587 106.8305) (end 126.492 104.9255) (width 0.3) (layer "F.Cu") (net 16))
 (via (at 124.587 112.268) (size 0.6) (drill 0.3) (layers "F.Cu" "B.Cu") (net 16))
 (via (at 124.587 118.11) (size 0.6) (drill 0.3) (layers "F.Cu" "B.Cu") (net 16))
 (segment (start 124.587 112.268) (end 124.587 118.11) (width 0.3) (layer "B.Cu") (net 16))
 (segment (start 121.539 106.299) (end 123.063 107.823) (width 0.3) (layer "F.Cu") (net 14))
 (segment (start 121.539 99.9725) (end 121.539 106.299) (width 0.3) (layer "F.Cu") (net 14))
 (segment (start 125.857 120.077) (end 125.857 118.11) (width 0.3) (layer "F.Cu") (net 14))
 (via (at 125.857 118.11) (size 0.6) (drill 0.3) (layers "F.Cu" "B.Cu") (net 14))
 (via (at 123.063 107.823) (size 0.6) (drill 0.3) (layers "F.Cu" "B.Cu") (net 14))
 (segment (start 125.476 110.236) (end 123.063 107.823) (width 0.3) (layer "B.Cu") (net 14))
 (segment (start 125.476 113.157) (end 125.476 110.236) (width 0.3) (layer "B.Cu") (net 14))
 (segment (start 125.842 118.095) (end 125.842 113.523) (width 0.3) (layer "B.Cu") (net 14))
 (segment (start 125.842 113.523) (end 125.476 113.157) (width 0.3) (layer "B.Cu") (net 14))
 (segment (start 125.857 118.11) (end 125.842 118.095) (width 0.3) (layer "B.Cu") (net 14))
 (segment (start 126.492 99.9725) (end 126.492 101.092) (width 0.3) (layer "F.Cu") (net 15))
 (segment (start 127.635 102.235) (end 127.635 107.569) (width 0.3) (layer "F.Cu") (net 15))
 (segment (start 127.635 107.569) (end 125.842 109.362) (width 0.3) (layer "F.Cu") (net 15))
 (segment (start 126.492 101.092) (end 127.635 102.235) (width 0.3) (layer "F.Cu") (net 15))
 (segment (start 125.842 115.112) (end 125.857 115.127) (width 0.3) (layer "F.Cu") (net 15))
 (segment (start 125.842 109.362) (end 125.842 115.112) (width 0.3) (layer "F.Cu") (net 15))
 (segment (start 121.539 95.0195) (end 121.539 96.52) (width 0.3) (layer "F.Cu") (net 4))
 (segment (start 124.587 113.665) (end 124.587 115.127) (width 0.3) (layer "F.Cu") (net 4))
 (segment (start 120.489 97.57) (end 120.489 109.567) (width 0.3) (layer "F.Cu") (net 4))
 (segment (start 120.489 109.567) (end 124.587 113.665) (width 0.3) (layer "F.Cu") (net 4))
 (segment (start 121.539 96.52) (end 120.489 97.57) (width 0.3) (layer "F.Cu") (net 4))
 (segment (start 127.127 112.776) (end 126.492 112.141) (width 0.3) (layer "F.Cu") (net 9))
 (segment (start 127.127 115.127) (end 127.127 112.776) (width 0.3) (layer "F.Cu") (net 9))
 (segment (start 126.492 95.0195) (end 126.492 96.52) (width 0.3) (layer "F.Cu") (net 9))
 (via (at 126.492 112.141) (size 0.6) (drill 0.3) (layers "F.Cu" "B.Cu") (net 9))
 (via (at 126.492 96.52) (size 0.6) (drill 0.3) (layers "F.Cu" "B.Cu") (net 9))
 (segment (start 126.492 96.52) (end 126.492 112.141) (width 0.3) (layer "B.Cu") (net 9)))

